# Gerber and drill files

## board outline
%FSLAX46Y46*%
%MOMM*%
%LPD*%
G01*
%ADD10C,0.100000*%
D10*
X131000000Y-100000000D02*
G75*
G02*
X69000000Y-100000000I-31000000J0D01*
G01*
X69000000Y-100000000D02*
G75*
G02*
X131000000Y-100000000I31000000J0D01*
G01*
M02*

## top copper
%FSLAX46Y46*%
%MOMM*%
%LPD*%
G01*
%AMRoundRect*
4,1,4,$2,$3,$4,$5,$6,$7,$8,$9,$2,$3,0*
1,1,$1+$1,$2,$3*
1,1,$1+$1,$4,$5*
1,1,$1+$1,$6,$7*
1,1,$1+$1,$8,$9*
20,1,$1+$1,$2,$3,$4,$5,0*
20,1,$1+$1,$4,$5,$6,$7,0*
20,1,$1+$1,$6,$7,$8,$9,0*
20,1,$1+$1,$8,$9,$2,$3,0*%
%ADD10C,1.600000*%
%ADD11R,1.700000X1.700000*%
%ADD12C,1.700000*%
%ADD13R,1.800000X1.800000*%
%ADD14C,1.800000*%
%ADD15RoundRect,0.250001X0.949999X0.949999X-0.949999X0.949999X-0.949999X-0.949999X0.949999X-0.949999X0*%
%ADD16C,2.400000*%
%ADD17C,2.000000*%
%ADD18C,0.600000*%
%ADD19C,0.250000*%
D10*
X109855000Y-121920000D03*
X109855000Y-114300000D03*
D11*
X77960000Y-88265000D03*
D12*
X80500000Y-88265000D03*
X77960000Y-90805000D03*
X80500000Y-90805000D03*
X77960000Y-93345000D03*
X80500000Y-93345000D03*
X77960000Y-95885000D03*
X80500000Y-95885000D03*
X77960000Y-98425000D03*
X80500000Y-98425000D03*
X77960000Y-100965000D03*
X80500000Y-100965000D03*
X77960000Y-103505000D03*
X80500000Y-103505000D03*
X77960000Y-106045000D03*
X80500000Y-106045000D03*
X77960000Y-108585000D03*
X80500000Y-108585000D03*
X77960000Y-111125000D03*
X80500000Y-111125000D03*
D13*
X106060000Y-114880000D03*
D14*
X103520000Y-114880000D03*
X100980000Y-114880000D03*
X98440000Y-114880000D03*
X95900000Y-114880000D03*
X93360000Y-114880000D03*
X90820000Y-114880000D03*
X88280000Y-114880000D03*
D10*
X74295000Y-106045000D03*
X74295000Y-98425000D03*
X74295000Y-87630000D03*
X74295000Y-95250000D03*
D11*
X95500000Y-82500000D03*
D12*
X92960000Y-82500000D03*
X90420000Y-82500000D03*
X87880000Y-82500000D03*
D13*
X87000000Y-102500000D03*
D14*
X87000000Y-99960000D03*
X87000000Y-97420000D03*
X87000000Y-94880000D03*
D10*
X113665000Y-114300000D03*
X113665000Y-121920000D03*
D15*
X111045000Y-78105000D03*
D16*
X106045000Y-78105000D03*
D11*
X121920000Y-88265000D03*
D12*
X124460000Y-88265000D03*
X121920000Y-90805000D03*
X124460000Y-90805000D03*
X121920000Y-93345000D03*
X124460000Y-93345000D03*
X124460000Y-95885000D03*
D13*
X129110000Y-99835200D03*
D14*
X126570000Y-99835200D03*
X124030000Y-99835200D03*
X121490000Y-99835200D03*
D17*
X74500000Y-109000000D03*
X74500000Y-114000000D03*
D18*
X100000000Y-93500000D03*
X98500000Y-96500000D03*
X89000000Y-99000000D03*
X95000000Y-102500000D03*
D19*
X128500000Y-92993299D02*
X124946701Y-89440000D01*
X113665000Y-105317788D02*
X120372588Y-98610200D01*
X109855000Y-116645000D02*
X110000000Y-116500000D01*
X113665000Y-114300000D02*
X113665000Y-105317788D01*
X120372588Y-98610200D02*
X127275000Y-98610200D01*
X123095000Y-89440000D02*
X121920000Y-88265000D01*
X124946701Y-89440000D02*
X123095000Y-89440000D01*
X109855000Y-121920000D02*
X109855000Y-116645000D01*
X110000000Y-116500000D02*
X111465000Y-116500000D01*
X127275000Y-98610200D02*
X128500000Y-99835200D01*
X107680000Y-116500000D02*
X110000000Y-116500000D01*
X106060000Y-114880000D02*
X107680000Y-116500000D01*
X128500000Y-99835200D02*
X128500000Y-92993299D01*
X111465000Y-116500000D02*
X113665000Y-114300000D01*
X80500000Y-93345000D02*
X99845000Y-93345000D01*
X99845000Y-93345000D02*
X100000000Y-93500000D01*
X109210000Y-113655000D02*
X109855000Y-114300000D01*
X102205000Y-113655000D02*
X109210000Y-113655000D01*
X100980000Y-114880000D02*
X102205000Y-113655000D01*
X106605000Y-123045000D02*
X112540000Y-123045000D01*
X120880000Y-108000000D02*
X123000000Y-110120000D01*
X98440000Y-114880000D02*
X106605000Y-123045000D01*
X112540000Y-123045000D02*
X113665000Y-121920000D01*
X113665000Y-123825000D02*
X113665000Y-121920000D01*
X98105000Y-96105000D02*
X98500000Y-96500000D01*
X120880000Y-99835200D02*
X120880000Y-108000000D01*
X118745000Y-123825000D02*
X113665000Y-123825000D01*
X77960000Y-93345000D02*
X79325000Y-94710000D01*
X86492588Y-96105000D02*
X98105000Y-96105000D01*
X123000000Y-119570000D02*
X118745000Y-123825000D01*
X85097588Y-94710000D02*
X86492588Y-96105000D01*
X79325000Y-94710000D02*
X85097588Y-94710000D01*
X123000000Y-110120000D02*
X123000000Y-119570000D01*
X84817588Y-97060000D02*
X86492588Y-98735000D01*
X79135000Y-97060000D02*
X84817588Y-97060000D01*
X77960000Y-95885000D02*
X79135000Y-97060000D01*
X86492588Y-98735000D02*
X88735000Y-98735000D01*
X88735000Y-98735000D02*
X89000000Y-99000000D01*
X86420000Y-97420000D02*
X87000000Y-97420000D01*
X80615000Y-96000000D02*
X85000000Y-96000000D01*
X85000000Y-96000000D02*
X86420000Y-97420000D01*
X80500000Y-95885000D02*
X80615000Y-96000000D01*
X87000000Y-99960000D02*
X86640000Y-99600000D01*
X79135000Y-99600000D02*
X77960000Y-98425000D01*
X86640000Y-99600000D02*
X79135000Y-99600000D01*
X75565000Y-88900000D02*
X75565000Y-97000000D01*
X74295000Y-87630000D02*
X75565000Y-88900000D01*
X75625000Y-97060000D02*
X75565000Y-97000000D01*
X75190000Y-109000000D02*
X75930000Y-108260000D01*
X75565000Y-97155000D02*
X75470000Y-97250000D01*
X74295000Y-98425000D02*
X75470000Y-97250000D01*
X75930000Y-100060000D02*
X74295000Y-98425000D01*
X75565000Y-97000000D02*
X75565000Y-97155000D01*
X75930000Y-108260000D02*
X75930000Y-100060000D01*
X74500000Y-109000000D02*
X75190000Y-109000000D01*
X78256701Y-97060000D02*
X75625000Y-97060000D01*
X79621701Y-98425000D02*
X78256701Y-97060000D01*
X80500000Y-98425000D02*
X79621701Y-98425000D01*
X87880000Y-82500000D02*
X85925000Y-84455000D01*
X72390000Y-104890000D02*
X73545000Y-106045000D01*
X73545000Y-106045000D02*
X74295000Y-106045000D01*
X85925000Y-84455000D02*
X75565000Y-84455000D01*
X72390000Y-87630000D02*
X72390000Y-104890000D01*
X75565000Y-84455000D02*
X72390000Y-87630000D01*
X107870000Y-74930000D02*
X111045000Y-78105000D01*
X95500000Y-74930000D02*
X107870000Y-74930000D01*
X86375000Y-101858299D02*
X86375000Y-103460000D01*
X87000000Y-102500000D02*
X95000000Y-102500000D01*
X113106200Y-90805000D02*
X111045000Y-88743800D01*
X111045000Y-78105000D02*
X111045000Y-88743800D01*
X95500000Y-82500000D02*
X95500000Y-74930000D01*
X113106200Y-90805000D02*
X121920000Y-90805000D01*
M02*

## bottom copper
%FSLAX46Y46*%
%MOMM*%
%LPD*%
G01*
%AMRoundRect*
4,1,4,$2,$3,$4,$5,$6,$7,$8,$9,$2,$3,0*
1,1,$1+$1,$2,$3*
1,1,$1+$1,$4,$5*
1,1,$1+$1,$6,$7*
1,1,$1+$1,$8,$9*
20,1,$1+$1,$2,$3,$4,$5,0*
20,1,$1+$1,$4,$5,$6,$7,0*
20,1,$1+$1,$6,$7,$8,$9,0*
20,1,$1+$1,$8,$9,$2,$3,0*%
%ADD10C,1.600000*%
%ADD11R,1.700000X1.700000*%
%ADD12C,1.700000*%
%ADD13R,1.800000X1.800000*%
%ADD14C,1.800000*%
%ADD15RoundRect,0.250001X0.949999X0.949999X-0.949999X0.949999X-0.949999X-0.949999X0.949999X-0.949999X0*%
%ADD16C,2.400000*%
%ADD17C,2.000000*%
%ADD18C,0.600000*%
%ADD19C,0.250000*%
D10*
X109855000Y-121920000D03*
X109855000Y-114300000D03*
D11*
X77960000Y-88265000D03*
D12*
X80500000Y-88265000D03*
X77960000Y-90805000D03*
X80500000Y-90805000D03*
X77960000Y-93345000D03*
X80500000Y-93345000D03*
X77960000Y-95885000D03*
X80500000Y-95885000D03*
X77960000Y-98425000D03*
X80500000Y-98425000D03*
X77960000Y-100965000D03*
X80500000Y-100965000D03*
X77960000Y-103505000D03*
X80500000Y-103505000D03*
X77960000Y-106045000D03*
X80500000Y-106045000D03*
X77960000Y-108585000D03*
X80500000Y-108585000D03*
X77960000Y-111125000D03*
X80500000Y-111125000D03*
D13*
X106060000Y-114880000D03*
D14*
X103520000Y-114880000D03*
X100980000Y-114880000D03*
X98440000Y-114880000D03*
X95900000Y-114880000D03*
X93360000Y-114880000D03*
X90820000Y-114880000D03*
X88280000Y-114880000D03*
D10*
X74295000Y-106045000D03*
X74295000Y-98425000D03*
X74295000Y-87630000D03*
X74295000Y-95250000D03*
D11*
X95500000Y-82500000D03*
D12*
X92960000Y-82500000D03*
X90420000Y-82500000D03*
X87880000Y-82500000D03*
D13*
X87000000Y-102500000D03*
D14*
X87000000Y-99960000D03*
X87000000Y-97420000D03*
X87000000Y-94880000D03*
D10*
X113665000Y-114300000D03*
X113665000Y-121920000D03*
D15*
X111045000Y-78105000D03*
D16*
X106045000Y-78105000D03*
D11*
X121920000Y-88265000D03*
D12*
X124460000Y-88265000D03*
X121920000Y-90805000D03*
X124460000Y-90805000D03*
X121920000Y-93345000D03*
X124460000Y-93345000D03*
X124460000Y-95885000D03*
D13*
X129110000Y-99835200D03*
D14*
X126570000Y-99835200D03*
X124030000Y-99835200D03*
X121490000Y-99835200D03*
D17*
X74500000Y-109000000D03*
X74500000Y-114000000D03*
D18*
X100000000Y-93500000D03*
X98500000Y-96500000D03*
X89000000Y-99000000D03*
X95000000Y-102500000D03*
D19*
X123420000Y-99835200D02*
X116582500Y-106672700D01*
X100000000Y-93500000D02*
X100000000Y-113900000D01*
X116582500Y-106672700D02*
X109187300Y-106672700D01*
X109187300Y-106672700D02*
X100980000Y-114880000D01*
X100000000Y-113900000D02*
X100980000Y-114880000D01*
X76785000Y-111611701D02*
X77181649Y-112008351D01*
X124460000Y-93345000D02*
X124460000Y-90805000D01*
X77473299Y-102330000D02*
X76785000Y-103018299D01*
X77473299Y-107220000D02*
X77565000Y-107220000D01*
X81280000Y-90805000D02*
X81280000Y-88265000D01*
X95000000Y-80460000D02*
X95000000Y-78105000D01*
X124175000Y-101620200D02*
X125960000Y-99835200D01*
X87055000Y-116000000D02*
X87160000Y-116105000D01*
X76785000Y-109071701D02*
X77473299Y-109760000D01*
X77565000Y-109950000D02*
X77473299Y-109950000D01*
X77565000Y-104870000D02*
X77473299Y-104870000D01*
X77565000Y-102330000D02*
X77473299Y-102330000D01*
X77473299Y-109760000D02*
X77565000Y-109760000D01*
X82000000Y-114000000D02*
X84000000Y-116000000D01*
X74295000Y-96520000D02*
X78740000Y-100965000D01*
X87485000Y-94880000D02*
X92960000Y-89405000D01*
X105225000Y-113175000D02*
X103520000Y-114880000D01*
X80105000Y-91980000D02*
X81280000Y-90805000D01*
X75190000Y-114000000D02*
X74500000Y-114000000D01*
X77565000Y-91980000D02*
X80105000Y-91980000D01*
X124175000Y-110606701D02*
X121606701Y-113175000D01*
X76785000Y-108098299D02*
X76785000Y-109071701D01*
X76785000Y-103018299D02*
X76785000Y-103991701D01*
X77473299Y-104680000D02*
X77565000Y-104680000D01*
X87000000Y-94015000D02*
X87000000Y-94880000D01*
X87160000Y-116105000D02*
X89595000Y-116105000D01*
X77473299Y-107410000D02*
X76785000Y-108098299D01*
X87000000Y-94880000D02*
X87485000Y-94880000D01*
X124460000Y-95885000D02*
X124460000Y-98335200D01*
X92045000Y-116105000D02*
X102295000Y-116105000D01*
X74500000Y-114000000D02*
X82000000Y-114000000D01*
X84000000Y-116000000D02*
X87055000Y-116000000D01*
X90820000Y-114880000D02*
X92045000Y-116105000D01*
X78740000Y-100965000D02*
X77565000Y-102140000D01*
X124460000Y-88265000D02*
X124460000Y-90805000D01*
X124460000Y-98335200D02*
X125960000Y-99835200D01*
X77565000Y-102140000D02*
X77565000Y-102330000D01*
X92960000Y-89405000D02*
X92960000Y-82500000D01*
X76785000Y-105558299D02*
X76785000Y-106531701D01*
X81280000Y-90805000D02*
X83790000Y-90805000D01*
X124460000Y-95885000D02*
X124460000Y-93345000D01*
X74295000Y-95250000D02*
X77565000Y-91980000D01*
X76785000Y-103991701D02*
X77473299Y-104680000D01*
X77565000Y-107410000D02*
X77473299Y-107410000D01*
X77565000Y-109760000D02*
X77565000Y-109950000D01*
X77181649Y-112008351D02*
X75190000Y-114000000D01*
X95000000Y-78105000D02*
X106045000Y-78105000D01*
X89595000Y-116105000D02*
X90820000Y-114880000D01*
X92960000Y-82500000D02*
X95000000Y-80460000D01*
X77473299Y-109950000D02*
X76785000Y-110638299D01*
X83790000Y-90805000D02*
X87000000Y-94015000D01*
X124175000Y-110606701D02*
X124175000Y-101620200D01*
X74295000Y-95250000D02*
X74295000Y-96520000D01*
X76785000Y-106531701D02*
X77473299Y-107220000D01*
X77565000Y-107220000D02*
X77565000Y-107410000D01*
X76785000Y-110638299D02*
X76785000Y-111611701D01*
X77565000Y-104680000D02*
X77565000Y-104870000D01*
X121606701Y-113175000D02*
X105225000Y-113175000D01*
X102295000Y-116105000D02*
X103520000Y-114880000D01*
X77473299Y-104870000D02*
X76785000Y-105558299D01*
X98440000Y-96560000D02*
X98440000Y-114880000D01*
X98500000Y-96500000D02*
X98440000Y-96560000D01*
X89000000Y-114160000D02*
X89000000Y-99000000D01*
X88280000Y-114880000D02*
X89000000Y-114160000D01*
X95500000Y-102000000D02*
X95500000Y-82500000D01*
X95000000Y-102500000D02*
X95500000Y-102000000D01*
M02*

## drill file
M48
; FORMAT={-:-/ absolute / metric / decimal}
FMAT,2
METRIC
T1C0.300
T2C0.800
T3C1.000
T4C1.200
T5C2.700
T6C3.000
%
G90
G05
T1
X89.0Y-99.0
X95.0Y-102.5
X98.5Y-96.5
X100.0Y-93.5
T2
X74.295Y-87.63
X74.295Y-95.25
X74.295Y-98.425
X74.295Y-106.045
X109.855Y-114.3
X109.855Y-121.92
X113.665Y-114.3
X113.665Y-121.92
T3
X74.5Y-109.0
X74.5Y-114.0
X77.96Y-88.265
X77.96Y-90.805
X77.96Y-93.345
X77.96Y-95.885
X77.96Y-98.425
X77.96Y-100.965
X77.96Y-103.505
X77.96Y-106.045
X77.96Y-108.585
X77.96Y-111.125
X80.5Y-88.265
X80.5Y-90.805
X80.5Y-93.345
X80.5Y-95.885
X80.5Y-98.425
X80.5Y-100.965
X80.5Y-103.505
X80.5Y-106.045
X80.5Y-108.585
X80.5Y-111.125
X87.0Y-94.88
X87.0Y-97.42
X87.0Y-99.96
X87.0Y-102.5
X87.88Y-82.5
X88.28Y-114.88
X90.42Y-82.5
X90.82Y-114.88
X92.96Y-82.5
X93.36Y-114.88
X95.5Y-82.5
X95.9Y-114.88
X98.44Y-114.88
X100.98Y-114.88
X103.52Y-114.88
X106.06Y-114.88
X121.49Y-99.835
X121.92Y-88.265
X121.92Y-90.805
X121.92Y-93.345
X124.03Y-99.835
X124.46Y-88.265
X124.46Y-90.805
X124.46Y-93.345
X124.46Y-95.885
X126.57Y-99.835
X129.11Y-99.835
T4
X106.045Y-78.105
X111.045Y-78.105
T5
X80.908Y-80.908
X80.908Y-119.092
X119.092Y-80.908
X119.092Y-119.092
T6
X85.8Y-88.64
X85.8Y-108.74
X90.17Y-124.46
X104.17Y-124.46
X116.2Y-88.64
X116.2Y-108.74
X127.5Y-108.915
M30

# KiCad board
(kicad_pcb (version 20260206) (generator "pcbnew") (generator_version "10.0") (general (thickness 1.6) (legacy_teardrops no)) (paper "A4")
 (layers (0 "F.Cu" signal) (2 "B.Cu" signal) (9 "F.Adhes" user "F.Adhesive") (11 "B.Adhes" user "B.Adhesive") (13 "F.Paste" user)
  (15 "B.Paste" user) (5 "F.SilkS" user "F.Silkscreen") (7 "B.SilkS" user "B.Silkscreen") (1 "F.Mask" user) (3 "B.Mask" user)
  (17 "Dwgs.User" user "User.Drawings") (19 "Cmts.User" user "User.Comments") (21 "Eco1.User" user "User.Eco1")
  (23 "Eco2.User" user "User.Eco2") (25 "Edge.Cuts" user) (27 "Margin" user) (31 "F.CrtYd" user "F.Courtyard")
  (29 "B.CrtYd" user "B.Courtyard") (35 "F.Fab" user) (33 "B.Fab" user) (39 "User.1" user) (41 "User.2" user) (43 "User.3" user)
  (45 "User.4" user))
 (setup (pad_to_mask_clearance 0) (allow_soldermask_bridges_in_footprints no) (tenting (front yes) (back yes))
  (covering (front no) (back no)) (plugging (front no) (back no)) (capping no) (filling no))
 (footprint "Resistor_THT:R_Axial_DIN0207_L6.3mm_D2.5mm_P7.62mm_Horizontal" (layer "F.Cu") (at 109.855 121.92 90)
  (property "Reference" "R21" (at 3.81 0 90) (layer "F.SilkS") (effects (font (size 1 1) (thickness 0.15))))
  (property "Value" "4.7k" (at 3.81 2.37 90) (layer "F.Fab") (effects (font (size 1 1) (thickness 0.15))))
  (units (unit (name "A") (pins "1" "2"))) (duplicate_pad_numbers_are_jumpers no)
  (pad "1" thru_hole circle (at 0 0 90) (size 1.6 1.6) (drill 0.8) (layers "*.Cu" "*.Mask") (remove_unused_layers no) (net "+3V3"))
  (pad "2" thru_hole circle (at 7.62 0 90) (size 1.6 1.6) (drill 0.8) (layers "*.Cu" "*.Mask") (remove_unused_layers no) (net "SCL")))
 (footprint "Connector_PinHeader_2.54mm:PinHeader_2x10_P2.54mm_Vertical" (layer "F.Cu") (at 77.96 88.265)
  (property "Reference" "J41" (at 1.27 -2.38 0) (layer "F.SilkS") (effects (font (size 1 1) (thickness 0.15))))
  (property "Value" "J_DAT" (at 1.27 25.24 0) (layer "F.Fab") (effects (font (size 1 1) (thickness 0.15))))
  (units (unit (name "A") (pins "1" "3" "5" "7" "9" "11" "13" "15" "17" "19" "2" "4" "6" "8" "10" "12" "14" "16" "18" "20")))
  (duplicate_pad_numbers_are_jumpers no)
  (pad "1" thru_hole rect (at 0 0) (size 1.7 1.7) (drill 1) (layers "*.Cu" "*.Mask") (remove_unused_layers no)
   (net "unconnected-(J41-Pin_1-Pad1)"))
  (pad "2" thru_hole circle (at 2.54 0) (size 1.7 1.7) (drill 1) (layers "*.Cu" "*.Mask") (remove_unused_layers no) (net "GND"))
  (pad "3" thru_hole circle (at 0 2.54) (size 1.7 1.7) (drill 1) (layers "*.Cu" "*.Mask") (remove_unused_layers no)
   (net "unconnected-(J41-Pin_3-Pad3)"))
  (pad "4" thru_hole circle (at 2.54 2.54) (size 1.7 1.7) (drill 1) (layers "*.Cu" "*.Mask") (remove_unused_layers no) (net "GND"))
  (pad "5" thru_hole circle (at 0 5.08) (size 1.7 1.7) (drill 1) (layers "*.Cu" "*.Mask") (remove_unused_layers no) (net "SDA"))
  (pad "6" thru_hole circle (at 2.54 5.08) (size 1.7 1.7) (drill 1) (layers "*.Cu" "*.Mask") (remove_unused_layers no) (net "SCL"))
  (pad "7" thru_hole circle (at 0 7.62) (size 1.7 1.7) (drill 1) (layers "*.Cu" "*.Mask") (remove_unused_layers no) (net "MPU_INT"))
  (pad "8" thru_hole circle (at 2.54 7.62) (size 1.7 1.7) (drill 1) (layers "*.Cu" "*.Mask") (remove_unused_layers no) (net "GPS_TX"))
  (pad "9" thru_hole circle (at 0 10.16) (size 1.7 1.7) (drill 1) (layers "*.Cu" "*.Mask") (remove_unused_layers no) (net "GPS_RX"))
  (pad "10" thru_hole circle (at 2.54 10.16) (size 1.7 1.7) (drill 1) (layers "*.Cu" "*.Mask") (remove_unused_layers no) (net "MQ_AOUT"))
  (pad "11" thru_hole circle (at 0 12.7) (size 1.7 1.7) (drill 1) (layers "*.Cu" "*.Mask") (remove_unused_layers no) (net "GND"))
  (pad "12" thru_hole circle (at 2.54 12.7) (size 1.7 1.7) (drill 1) (layers "*.Cu" "*.Mask") (remove_unused_layers no)
   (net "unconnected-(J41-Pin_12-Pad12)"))
  (pad "13" thru_hole circle (at 0 15.24) (size 1.7 1.7) (drill 1) (layers "*.Cu" "*.Mask") (remove_unused_layers no)
   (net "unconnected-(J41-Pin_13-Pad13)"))
  (pad "14" thru_hole circle (at 2.54 15.24) (size 1.7 1.7) (drill 1) (layers "*.Cu" "*.Mask") (remove_unused_layers no)
   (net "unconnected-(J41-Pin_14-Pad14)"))
  (pad "15" thru_hole circle (at 0 17.78) (size 1.7 1.7) (drill 1) (layers "*.Cu" "*.Mask") (remove_unused_layers no)
   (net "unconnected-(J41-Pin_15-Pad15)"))
  (pad "16" thru_hole circle (at 2.54 17.78) (size 1.7 1.7) (drill 1) (layers "*.Cu" "*.Mask") (remove_unused_layers no)
   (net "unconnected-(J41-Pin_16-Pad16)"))
  (pad "17" thru_hole circle (at 0 20.32) (size 1.7 1.7) (drill 1) (layers "*.Cu" "*.Mask") (remove_unused_layers no)
   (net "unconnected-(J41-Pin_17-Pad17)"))
  (pad "18" thru_hole circle (at 2.54 20.32) (size 1.7 1.7) (drill 1) (layers "*.Cu" "*.Mask") (remove_unused_layers no)
   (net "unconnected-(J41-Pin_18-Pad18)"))
  (pad "19" thru_hole circle (at 0 22.86) (size 1.7 1.7) (drill 1) (layers "*.Cu" "*.Mask") (remove_unused_layers no)
   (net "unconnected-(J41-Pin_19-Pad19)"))
  (pad "20" thru_hole circle (at 2.54 22.86) (size 1.7 1.7) (drill 1) (layers "*.Cu" "*.Mask") (remove_unused_layers no)
   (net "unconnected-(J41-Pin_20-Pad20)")))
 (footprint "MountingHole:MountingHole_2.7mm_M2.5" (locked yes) (layer "F.Cu") (at 119.092 119.092)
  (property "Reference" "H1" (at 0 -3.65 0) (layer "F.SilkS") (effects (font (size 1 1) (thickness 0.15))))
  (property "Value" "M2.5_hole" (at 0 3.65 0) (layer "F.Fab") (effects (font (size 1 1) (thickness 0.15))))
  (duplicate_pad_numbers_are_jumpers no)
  (pad "" np_thru_hole circle (at 0 0) (size 2.7 2.7) (drill 2.7) (layers "*.Cu" "*.Mask")))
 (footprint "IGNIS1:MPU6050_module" (layer "F.Cu") (at 97.17 119.96 -90)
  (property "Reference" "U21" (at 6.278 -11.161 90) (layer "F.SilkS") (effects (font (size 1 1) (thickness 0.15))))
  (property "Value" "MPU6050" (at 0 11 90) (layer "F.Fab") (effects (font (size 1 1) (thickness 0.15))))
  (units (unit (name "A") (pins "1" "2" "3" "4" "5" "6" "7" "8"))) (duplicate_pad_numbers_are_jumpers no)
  (pad "" np_thru_hole circle (at 4.5 -7 270) (size 3 3) (drill 3) (layers "*.Cu" "*.Mask"))
  (pad "" np_thru_hole circle (at 4.5 7 270) (size 3 3) (drill 3) (layers "*.Cu" "*.Mask"))
  (pad "1" thru_hole rect (at -5.08 -8.89 270) (size 1.8 1.8) (drill 1) (layers "*.Cu" "*.Mask") (remove_unused_layers no) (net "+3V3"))
  (pad "2" thru_hole circle (at -5.08 -6.35 270) (size 1.8 1.8) (drill 1) (layers "*.Cu" "*.Mask") (remove_unused_layers no) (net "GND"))
  (pad "3" thru_hole circle (at -5.08 -3.81 270) (size 1.8 1.8) (drill 1) (layers "*.Cu" "*.Mask") (remove_unused_layers no) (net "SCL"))
  (pad "4" thru_hole circle (at -5.08 -1.27 270) (size 1.8 1.8) (drill 1) (layers "*.Cu" "*.Mask") (remove_unused_layers no) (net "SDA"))
  (pad "5" thru_hole circle (at -5.08 1.27 270) (size 1.8 1.8) (drill 1) (layers "*.Cu" "*.Mask") (remove_unused_layers no)
   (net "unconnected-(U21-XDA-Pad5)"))
  (pad "6" thru_hole circle (at -5.08 3.81 270) (size 1.8 1.8) (drill 1) (layers "*.Cu" "*.Mask") (remove_unused_layers no)
   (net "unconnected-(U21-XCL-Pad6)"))
  (pad "7" thru_hole circle (at -5.08 6.35 270) (size 1.8 1.8) (drill 1) (layers "*.Cu" "*.Mask") (remove_unused_layers no) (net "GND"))
  (pad "8" thru_hole circle (at -5.08 8.89 270) (size 1.8 1.8) (drill 1) (layers "*.Cu" "*.Mask") (remove_unused_layers no) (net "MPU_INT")))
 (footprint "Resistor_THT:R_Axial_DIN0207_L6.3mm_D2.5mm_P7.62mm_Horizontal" (layer "F.Cu") (at 74.295 106.045 90)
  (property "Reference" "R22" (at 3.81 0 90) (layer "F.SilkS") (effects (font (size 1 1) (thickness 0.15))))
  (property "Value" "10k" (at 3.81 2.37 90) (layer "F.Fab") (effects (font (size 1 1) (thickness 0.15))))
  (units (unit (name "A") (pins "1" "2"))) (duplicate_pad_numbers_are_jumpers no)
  (pad "1" thru_hole circle (at 0 0 90) (size 1.6 1.6) (drill 0.8) (layers "*.Cu" "*.Mask") (remove_unused_layers no) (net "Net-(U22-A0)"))
  (pad "2" thru_hole circle (at 7.62 0 90) (size 1.6 1.6) (drill 0.8) (layers "*.Cu" "*.Mask") (remove_unused_layers no) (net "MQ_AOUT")))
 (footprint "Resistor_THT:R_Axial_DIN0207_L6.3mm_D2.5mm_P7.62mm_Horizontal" (layer "F.Cu") (at 74.295 87.63 -90)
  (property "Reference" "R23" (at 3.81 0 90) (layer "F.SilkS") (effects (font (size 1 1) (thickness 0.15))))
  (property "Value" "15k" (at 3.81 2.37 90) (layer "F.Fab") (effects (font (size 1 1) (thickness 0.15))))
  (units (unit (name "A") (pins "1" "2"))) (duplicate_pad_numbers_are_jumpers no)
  (pad "1" thru_hole circle (at 0 0 270) (size 1.6 1.6) (drill 0.8) (layers "*.Cu" "*.Mask") (remove_unused_layers no) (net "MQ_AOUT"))
  (pad "2" thru_hole circle (at 7.62 0 270) (size 1.6 1.6) (drill 0.8) (layers "*.Cu" "*.Mask") (remove_unused_layers no) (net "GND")))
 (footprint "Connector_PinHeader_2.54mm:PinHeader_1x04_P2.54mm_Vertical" (layer "F.Cu") (at 95.5 82.5 -90)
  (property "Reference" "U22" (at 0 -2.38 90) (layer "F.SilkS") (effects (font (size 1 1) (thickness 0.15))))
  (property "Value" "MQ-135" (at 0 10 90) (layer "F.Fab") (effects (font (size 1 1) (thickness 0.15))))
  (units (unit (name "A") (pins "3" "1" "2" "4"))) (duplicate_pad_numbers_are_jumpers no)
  (pad "1" thru_hole rect (at 0 0 270) (size 1.7 1.7) (drill 1) (layers "*.Cu" "*.Mask") (remove_unused_layers no) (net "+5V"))
  (pad "2" thru_hole circle (at 0 2.54 270) (size 1.7 1.7) (drill 1) (layers "*.Cu" "*.Mask") (remove_unused_layers no) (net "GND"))
  (pad "3" thru_hole circle (at 0 5.08 270) (size 1.7 1.7) (drill 1) (layers "*.Cu" "*.Mask") (remove_unused_layers no)
   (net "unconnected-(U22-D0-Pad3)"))
  (pad "4" thru_hole circle (at 0 7.62 270) (size 1.7 1.7) (drill 1) (layers "*.Cu" "*.Mask") (remove_unused_layers no) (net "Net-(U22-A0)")))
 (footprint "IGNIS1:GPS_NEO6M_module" (layer "F.Cu") (at 101 98.69)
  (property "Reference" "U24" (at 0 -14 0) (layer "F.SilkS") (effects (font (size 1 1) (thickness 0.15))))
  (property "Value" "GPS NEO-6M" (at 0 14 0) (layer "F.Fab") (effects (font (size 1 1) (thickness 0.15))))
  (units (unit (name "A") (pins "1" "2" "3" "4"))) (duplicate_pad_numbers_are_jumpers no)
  (pad "" np_thru_hole circle (at -15.2 -10.05) (size 3 3) (drill 3) (layers "*.Cu" "*.Mask"))
  (pad "" np_thru_hole circle (at -15.2 10.05) (size 3 3) (drill 3) (layers "*.Cu" "*.Mask"))
  (pad "" np_thru_hole circle (at 15.2 -10.05) (size 3 3) (drill 3) (layers "*.Cu" "*.Mask"))
  (pad "" np_thru_hole circle (at 15.2 10.05) (size 3 3) (drill 3) (layers "*.Cu" "*.Mask"))
  (pad "1" thru_hole rect (at -14 3.81) (size 1.8 1.8) (drill 1) (layers "*.Cu" "*.Mask") (remove_unused_layers no) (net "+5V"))
  (pad "2" thru_hole circle (at -14 1.27) (size 1.8 1.8) (drill 1) (layers "*.Cu" "*.Mask") (remove_unused_layers no) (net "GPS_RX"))
  (pad "3" thru_hole circle (at -14 -1.27) (size 1.8 1.8) (drill 1) (layers "*.Cu" "*.Mask") (remove_unused_layers no) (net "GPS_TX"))
  (pad "4" thru_hole circle (at -14 -3.81) (size 1.8 1.8) (drill 1) (layers "*.Cu" "*.Mask") (remove_unused_layers no) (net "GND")))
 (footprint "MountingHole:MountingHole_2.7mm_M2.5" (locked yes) (layer "F.Cu") (at 80.908 80.908)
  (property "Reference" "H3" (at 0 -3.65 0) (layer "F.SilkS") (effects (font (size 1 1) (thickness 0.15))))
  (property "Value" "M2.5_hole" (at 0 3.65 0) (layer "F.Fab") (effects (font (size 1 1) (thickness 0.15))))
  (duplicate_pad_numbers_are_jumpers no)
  (pad "" np_thru_hole circle (at 0 0) (size 2.7 2.7) (drill 2.7) (layers "*.Cu" "*.Mask")))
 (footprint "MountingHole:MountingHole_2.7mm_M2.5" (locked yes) (layer "F.Cu") (at 119.092 80.908)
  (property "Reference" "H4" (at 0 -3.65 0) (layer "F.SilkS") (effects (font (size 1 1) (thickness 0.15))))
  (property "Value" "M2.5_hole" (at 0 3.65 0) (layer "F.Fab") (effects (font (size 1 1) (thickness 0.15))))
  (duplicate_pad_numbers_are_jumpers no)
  (pad "" np_thru_hole circle (at 0 0) (size 2.7 2.7) (drill 2.7) (layers "*.Cu" "*.Mask")))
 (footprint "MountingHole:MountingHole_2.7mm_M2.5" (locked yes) (layer "F.Cu") (at 80.908 119.092)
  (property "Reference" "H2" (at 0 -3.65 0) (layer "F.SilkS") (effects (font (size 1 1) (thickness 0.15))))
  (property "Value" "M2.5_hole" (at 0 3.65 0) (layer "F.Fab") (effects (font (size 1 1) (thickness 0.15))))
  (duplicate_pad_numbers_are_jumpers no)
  (pad "" np_thru_hole circle (at 0 0) (size 2.7 2.7) (drill 2.7) (layers "*.Cu" "*.Mask")))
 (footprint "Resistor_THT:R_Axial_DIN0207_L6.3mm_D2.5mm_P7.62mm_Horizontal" (layer "F.Cu") (at 113.665 114.3 -90)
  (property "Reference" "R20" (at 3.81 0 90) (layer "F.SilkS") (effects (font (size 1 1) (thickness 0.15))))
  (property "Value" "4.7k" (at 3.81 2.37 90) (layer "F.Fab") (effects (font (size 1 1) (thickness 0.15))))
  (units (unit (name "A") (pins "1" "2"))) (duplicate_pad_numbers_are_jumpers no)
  (pad "1" thru_hole circle (at 0 0 270) (size 1.6 1.6) (drill 0.8) (layers "*.Cu" "*.Mask") (remove_unused_layers no) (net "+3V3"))
  (pad "2" thru_hole circle (at 7.62 0 270) (size 1.6 1.6) (drill 0.8) (layers "*.Cu" "*.Mask") (remove_unused_layers no) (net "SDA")))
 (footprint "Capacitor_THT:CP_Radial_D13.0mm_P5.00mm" (layer "F.Cu") (at 111.045 78.105 180)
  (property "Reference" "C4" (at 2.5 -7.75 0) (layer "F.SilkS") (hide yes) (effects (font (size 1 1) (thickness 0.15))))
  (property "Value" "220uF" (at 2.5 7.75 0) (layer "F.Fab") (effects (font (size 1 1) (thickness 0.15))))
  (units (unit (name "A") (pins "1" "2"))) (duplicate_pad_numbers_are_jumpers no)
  (pad "1" thru_hole roundrect (at 0 0 180) (size 2.4 2.4) (drill 1.2) (layers "*.Cu" "*.Mask") (remove_unused_layers no)
   (roundrect_rratio 0.104167) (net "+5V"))
  (pad "2" thru_hole circle (at 5 0 180) (size 2.4 2.4) (drill 1.2) (layers "*.Cu" "*.Mask") (remove_unused_layers no) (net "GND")))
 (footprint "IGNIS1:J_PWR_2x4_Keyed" (layer "F.Cu") (at 123.19 92.075)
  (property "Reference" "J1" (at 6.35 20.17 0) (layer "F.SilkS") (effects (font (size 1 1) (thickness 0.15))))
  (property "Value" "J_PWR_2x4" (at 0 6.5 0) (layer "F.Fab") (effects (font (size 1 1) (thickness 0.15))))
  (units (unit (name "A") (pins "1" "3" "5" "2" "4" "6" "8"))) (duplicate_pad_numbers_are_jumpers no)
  (pad "1" thru_hole rect (at -1.27 -3.81) (size 1.7 1.7) (drill 1) (layers "*.Cu" "*.Mask") (remove_unused_layers no) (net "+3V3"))
  (pad "2" thru_hole circle (at 1.27 -3.81) (size 1.7 1.7) (drill 1) (layers "*.Cu" "*.Mask") (remove_unused_layers no) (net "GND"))
  (pad "3" thru_hole circle (at -1.27 -1.27) (size 1.7 1.7) (drill 1) (layers "*.Cu" "*.Mask") (remove_unused_layers no) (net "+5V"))
  (pad "4" thru_hole circle (at 1.27 -1.27) (size 1.7 1.7) (drill 1) (layers "*.Cu" "*.Mask") (remove_unused_layers no) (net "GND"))
  (pad "5" thru_hole circle (at -1.27 1.27) (size 1.7 1.7) (drill 1) (layers "*.Cu" "*.Mask") (remove_unused_layers no)
   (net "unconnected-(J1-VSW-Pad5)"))
  (pad "6" thru_hole circle (at 1.27 1.27) (size 1.7 1.7) (drill 1) (layers "*.Cu" "*.Mask") (remove_unused_layers no) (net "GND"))
  (pad "8" thru_hole circle (at 1.27 3.81) (size 1.7 1.7) (drill 1) (layers "*.Cu" "*.Mask") (remove_unused_layers no) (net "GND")))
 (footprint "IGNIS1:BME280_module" (layer "F.Cu") (at 125.3 104.9152 -90)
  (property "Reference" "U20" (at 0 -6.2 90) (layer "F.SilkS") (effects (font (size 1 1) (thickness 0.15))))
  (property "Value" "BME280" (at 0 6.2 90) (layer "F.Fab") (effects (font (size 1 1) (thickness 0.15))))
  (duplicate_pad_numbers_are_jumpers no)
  (pad "" np_thru_hole circle (at 4 -2.2 270) (size 3 3) (drill 3) (layers "*.Cu" "*.Mask"))
  (pad "1" thru_hole rect (at -5.08 -3.81 270) (size 1.8 1.8) (drill 1) (layers "*.Cu" "*.Mask") (remove_unused_layers no) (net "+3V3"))
  (pad "2" thru_hole circle (at -5.08 -1.27 270) (size 1.8 1.8) (drill 1) (layers "*.Cu" "*.Mask") (remove_unused_layers no) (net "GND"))
  (pad "3" thru_hole circle (at -5.08 1.27 270) (size 1.8 1.8) (drill 1) (layers "*.Cu" "*.Mask") (remove_unused_layers no) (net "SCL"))
  (pad "4" thru_hole circle (at -5.08 3.81 270) (size 1.8 1.8) (drill 1) (layers "*.Cu" "*.Mask") (remove_unused_layers no) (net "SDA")))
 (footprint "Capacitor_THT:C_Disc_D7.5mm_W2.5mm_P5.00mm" (layer "F.Cu") (at 74.5 109 -90)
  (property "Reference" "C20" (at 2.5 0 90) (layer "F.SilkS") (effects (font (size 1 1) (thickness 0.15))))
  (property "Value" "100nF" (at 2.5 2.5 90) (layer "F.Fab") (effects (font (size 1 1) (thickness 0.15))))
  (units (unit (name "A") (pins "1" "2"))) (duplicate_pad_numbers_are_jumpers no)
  (pad "1" thru_hole circle (at 0 0 270) (size 2 2) (drill 1) (layers "*.Cu" "*.Mask") (remove_unused_layers no) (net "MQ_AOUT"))
  (pad "2" thru_hole circle (at 5 0 270) (size 2 2) (drill 1) (layers "*.Cu" "*.Mask") (remove_unused_layers no) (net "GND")))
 (gr_circle (center 100 100) (end 131 100) (stroke (width 0.1) (type solid)) (fill no) (locked yes) (layer "Edge.Cuts"))
 (segment (start 128.5 92.993299) (end 124.946701 89.44) (width 0.25) (layer "F.Cu") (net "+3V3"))
 (segment (start 113.665 105.317788) (end 120.372588 98.6102) (width 0.25) (layer "F.Cu") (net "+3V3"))
 (segment (start 109.855 116.645) (end 110 116.5) (width 0.25) (layer "F.Cu") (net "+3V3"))
 (segment (start 113.665 114.3) (end 113.665 105.317788) (width 0.25) (layer "F.Cu") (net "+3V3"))
 (segment (start 120.372588 98.6102) (end 127.275 98.6102) (width 0.25) (layer "F.Cu") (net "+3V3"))
 (segment (start 123.095 89.44) (end 121.92 88.265) (width 0.25) (layer "F.Cu") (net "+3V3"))
 (segment (start 124.946701 89.44) (end 123.095 89.44) (width 0.25) (layer "F.Cu") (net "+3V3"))
 (segment (start 109.855 121.92) (end 109.855 116.645) (width 0.25) (layer "F.Cu") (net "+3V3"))
 (segment (start 110 116.5) (end 111.465 116.5) (width 0.25) (layer "F.Cu") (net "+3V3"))
 (segment (start 127.275 98.6102) (end 128.5 99.8352) (width 0.25) (layer "F.Cu") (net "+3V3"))
 (segment (start 107.68 116.5) (end 110 116.5) (width 0.25) (layer "F.Cu") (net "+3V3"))
 (segment (start 106.06 114.88) (end 107.68 116.5) (width 0.25) (layer "F.Cu") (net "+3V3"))
 (segment (start 128.5 99.8352) (end 128.5 92.993299) (width 0.25) (layer "F.Cu") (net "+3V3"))
 (segment (start 111.465 116.5) (end 113.665 114.3) (width 0.25) (layer "F.Cu") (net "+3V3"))
 (segment (start 80.5 93.345) (end 99.845 93.345) (width 0.25) (layer "F.Cu") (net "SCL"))
 (segment (start 99.845 93.345) (end 100 93.5) (width 0.25) (layer "F.Cu") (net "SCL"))
 (segment (start 109.21 113.655) (end 109.855 114.3) (width 0.25) (layer "F.Cu") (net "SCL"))
 (segment (start 102.205 113.655) (end 109.21 113.655) (width 0.25) (layer "F.Cu") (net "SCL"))
 (segment (start 100.98 114.88) (end 102.205 113.655) (width 0.25) (layer "F.Cu") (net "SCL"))
 (via (at 100 93.5) (size 0.6) (drill 0.3) (layers "F.Cu" "B.Cu") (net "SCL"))
 (segment (start 123.42 99.8352) (end 116.5825 106.6727) (width 0.25) (layer "B.Cu") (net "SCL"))
 (segment (start 100 93.5) (end 100 113.9) (width 0.25) (layer "B.Cu") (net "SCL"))
 (segment (start 116.5825 106.6727) (end 109.1873 106.6727) (width 0.25) (layer "B.Cu") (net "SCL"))
 (segment (start 109.1873 106.6727) (end 100.98 114.88) (width 0.25) (layer "B.Cu") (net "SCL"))
 (segment (start 100 113.9) (end 100.98 114.88) (width 0.25) (layer "B.Cu") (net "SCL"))
 (segment (start 76.785 111.611701) (end 77.181649 112.008351) (width 0.25) (layer "B.Cu") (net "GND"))
 (segment (start 124.46 93.345) (end 124.46 90.805) (width 0.25) (layer "B.Cu") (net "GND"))
 (segment (start 77.473299 102.33) (end 76.785 103.018299) (width 0.25) (layer "B.Cu") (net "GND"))
 (segment (start 77.473299 107.22) (end 77.565 107.22) (width 0.25) (layer "B.Cu") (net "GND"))
 (segment (start 81.28 90.805) (end 81.28 88.265) (width 0.25) (layer "B.Cu") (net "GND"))
 (segment (start 95 80.46) (end 95 78.105) (width 0.25) (layer "B.Cu") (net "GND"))
 (segment (start 124.175 101.6202) (end 125.96 99.8352) (width 0.25) (layer "B.Cu") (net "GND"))
 (segment (start 87.055 116) (end 87.16 116.105) (width 0.25) (layer "B.Cu") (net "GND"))
 (segment (start 76.785 109.071701) (end 77.473299 109.76) (width 0.25) (layer "B.Cu") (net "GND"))
 (segment (start 77.565 109.95) (end 77.473299 109.95) (width 0.25) (layer "B.Cu") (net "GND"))
 (segment (start 77.565 104.87) (end 77.473299 104.87) (width 0.25) (layer "B.Cu") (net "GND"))
 (segment (start 77.565 102.33) (end 77.473299 102.33) (width 0.25) (layer "B.Cu") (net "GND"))
 (segment (start 77.473299 109.76) (end 77.565 109.76) (width 0.25) (layer "B.Cu") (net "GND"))
 (segment (start 82 114) (end 84 116) (width 0.25) (layer "B.Cu") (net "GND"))
 (segment (start 74.295 96.52) (end 78.74 100.965) (width 0.25) (layer "B.Cu") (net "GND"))
 (segment (start 87.485 94.88) (end 92.96 89.405) (width 0.25) (layer "B.Cu") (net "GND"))
 (segment (start 105.225 113.175) (end 103.52 114.88) (width 0.25) (layer "B.Cu") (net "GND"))
 (segment (start 80.105 91.98) (end 81.28 90.805) (width 0.25) (layer "B.Cu") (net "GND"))
 (segment (start 75.19 114) (end 74.5 114) (width 0.25) (layer "B.Cu") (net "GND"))
 (segment (start 77.565 91.98) (end 80.105 91.98) (width 0.25) (layer "B.Cu") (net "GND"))
 (segment (start 124.175 110.606701) (end 121.606701 113.175) (width 0.25) (layer "B.Cu") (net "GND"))
 (segment (start 76.785 108.098299) (end 76.785 109.071701) (width 0.25) (layer "B.Cu") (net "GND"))
 (segment (start 76.785 103.018299) (end 76.785 103.991701) (width 0.25) (layer "B.Cu") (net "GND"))
 (segment (start 77.473299 104.68) (end 77.565 104.68) (width 0.25) (layer "B.Cu") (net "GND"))
 (segment (start 87 94.015) (end 87 94.88) (width 0.25) (layer "B.Cu") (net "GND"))
 (segment (start 87.16 116.105) (end 89.595 116.105) (width 0.25) (layer "B.Cu") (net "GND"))
 (segment (start 77.473299 107.41) (end 76.785 108.098299) (width 0.25) (layer "B.Cu") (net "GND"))
 (segment (start 87 94.88) (end 87.485 94.88) (width 0.25) (layer "B.Cu") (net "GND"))
 (segment (start 124.46 95.885) (end 124.46 98.3352) (width 0.25) (layer "B.Cu") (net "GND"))
 (segment (start 92.045 116.105) (end 102.295 116.105) (width 0.25) (layer "B.Cu") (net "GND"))
 (segment (start 74.5 114) (end 82 114) (width 0.25) (layer "B.Cu") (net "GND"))
 (segment (start 84 116) (end 87.055 116) (width 0.25) (layer "B.Cu") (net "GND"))
 (segment (start 90.82 114.88) (end 92.045 116.105) (width 0.25) (layer "B.Cu") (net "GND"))
 (segment (start 78.74 100.965) (end 77.565 102.14) (width 0.25) (layer "B.Cu") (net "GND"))
 (segment (start 124.46 88.265) (end 124.46 90.805) (width 0.25) (layer "B.Cu") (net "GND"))
 (segment (start 124.46 98.3352) (end 125.96 99.8352) (width 0.25) (layer "B.Cu") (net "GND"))
 (segment (start 77.565 102.14) (end 77.565 102.33) (width 0.25) (layer "B.Cu") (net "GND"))
 (segment (start 92.96 89.405) (end 92.96 82.5) (width 0.25) (layer "B.Cu") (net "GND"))
 (segment (start 76.785 105.558299) (end 76.785 106.531701) (width 0.25) (layer "B.Cu") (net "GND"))
 (segment (start 81.28 90.805) (end 83.79 90.805) (width 0.25) (layer "B.Cu") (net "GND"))
 (segment (start 124.46 95.885) (end 124.46 93.345) (width 0.25) (layer "B.Cu") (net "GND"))
 (segment (start 74.295 95.25) (end 77.565 91.98) (width 0.25) (layer "B.Cu") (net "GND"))
 (segment (start 76.785 103.991701) (end 77.473299 104.68) (width 0.25) (layer "B.Cu") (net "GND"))
 (segment (start 77.565 107.41) (end 77.473299 107.41) (width 0.25) (layer "B.Cu") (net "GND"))
 (segment (start 77.565 109.76) (end 77.565 109.95) (width 0.25) (layer "B.Cu") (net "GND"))
 (segment (start 77.181649 112.008351) (end 75.19 114) (width 0.25) (layer "B.Cu") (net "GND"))
 (segment (start 95 78.105) (end 106.045 78.105) (width 0.25) (layer "B.Cu") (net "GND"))
 (segment (start 89.595 116.105) (end 90.82 114.88) (width 0.25) (layer "B.Cu") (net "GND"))
 (segment (start 92.96 82.5) (end 95 80.46) (width 0.25) (layer "B.Cu") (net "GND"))
 (segment (start 77.473299 109.95) (end 76.785 110.638299) (width 0.25) (layer "B.Cu") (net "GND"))
 (segment (start 83.79 90.805) (end 87 94.015) (width 0.25) (layer "B.Cu") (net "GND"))
 (segment (start 124.175 110.606701) (end 124.175 101.6202) (width 0.25) (layer "B.Cu") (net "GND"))
 (segment (start 74.295 95.25) (end 74.295 96.52) (width 0.25) (layer "B.Cu") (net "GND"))
 (segment (start 76.785 106.531701) (end 77.473299 107.22) (width 0.25) (layer "B.Cu") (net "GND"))
 (segment (start 77.565 107.22) (end 77.565 107.41) (width 0.25) (layer "B.Cu") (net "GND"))
 (segment (start 76.785 110.638299) (end 76.785 111.611701) (width 0.25) (layer "B.Cu") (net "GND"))
 (segment (start 77.565 104.68) (end 77.565 104.87) (width 0.25) (layer "B.Cu") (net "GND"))
 (segment (start 121.606701 113.175) (end 105.225 113.175) (width 0.25) (layer "B.Cu") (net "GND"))
 (segment (start 102.295 116.105) (end 103.52 114.88) (width 0.25) (layer "B.Cu") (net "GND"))
 (segment (start 77.473299 104.87) (end 76.785 105.558299) (width 0.25) (layer "B.Cu") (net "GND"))
 (segment (start 106.605 123.045) (end 112.54 123.045) (width 0.25) (layer "F.Cu") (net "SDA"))
 (segment (start 120.88 108) (end 123 110.12) (width 0.25) (layer "F.Cu") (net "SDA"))
 (segment (start 98.44 114.88) (end 106.605 123.045) (width 0.25) (layer "F.Cu") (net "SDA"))
 (segment (start 112.54 123.045) (end 113.665 121.92) (width 0.25) (layer "F.Cu") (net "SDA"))
 (segment (start 113.665 123.825) (end 113.665 121.92) (width 0.25) (layer "F.Cu") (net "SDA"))
 (segment (start 98.105 96.105) (end 98.5 96.5) (width 0.25) (layer "F.Cu") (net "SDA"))
 (segment (start 120.88 99.8352) (end 120.88 108) (width 0.25) (layer "F.Cu") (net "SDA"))
 (segment (start 118.745 123.825) (end 113.665 123.825) (width 0.25) (layer "F.Cu") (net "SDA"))
 (segment (start 77.96 93.345) (end 79.325 94.71) (width 0.25) (layer "F.Cu") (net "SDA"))
 (segment (start 86.492588 96.105) (end 98.105 96.105) (width 0.25) (layer "F.Cu") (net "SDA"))
 (segment (start 123 119.57) (end 118.745 123.825) (width 0.25) (layer "F.Cu") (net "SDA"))
 (segment (start 85.097588 94.71) (end 86.492588 96.105) (width 0.25) (layer "F.Cu") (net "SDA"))
 (segment (start 79.325 94.71) (end 85.097588 94.71) (width 0.25) (layer "F.Cu") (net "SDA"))
 (segment (start 123 110.12) (end 123 119.57) (width 0.25) (layer "F.Cu") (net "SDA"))
 (via (at 98.5 96.5) (size 0.6) (drill 0.3) (layers "F.Cu" "B.Cu") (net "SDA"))
 (segment (start 98.44 96.56) (end 98.44 114.88) (width 0.25) (layer "B.Cu") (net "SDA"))
 (segment (start 98.5 96.5) (end 98.44 96.56) (width 0.25) (layer "B.Cu") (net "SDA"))
 (segment (start 84.817588 97.06) (end 86.492588 98.735) (width 0.25) (layer "F.Cu") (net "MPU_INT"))
 (segment (start 79.135 97.06) (end 84.817588 97.06) (width 0.25) (layer "F.Cu") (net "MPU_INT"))
 (segment (start 77.96 95.885) (end 79.135 97.06) (width 0.25) (layer "F.Cu") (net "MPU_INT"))
 (segment (start 86.492588 98.735) (end 88.735 98.735) (width 0.25) (layer "F.Cu") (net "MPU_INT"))
 (segment (start 88.735 98.735) (end 89 99) (width 0.25) (layer "F.Cu") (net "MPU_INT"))
 (via (at 89 99) (size 0.6) (drill 0.3) (layers "F.Cu" "B.Cu") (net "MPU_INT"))
 (segment (start 89 114.16) (end 89 99) (width 0.25) (layer "B.Cu") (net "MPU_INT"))
 (segment (start 88.28 114.88) (end 89 114.16) (width 0.25) (layer "B.Cu") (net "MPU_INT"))
 (segment (start 86.42 97.42) (end 87 97.42) (width 0.25) (layer "F.Cu") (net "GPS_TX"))
 (segment (start 80.615 96) (end 85 96) (width 0.25) (layer "F.Cu") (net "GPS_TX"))
 (segment (start 85 96) (end 86.42 97.42) (width 0.25) (layer "F.Cu") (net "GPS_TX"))
 (segment (start 80.5 95.885) (end 80.615 96) (width 0.25) (layer "F.Cu") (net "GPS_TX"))
 (segment (start 87 99.96) (end 86.64 99.6) (width 0.25) (layer "F.Cu") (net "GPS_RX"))
 (segment (start 79.135 99.6) (end 77.96 98.425) (width 0.25) (layer "F.Cu") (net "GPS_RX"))
 (segment (start 86.64 99.6) (end 79.135 99.6) (width 0.25) (layer "F.Cu") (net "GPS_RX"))
 (segment (start 75.565 88.9) (end 75.565 97) (width 0.25) (layer "F.Cu") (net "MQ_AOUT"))
 (segment (start 74.295 87.63) (end 75.565 88.9) (width 0.25) (layer "F.Cu") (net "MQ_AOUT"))
 (segment (start 75.625 97.06) (end 75.565 97) (width 0.25) (layer "F.Cu") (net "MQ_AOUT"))
 (segment (start 75.19 109) (end 75.93 108.26) (width 0.25) (layer "F.Cu") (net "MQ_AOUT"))
 (segment (start 75.565 97.155) (end 75.47 97.25) (width 0.25) (layer "F.Cu") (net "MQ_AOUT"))
 (segment (start 74.295 98.425) (end 75.47 97.25) (width 0.25) (layer "F.Cu") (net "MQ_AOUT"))
 (segment (start 75.93 100.06) (end 74.295 98.425) (width 0.25) (layer "F.Cu") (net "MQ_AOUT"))
 (segment (start 75.565 97) (end 75.565 97.155) (width 0.25) (layer "F.Cu") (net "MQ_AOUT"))
 (segment (start 75.93 108.26) (end 75.93 100.06) (width 0.25) (layer "F.Cu") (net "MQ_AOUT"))
 (segment (start 74.5 109) (end 75.19 109) (width 0.25) (layer "F.Cu") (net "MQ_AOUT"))
 (segment (start 78.256701 97.06) (end 75.625 97.06) (width 0.25) (layer "F.Cu") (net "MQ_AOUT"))
 (segment (start 79.621701 98.425) (end 78.256701 97.06) (width 0.25) (layer "F.Cu") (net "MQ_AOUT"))
 (segment (start 80.5 98.425) (end 79.621701 98.425) (width 0.25) (layer "F.Cu") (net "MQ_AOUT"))
 (segment (start 87.88 82.5) (end 85.925 84.455) (width 0.25) (layer "F.Cu") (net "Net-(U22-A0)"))
 (segment (start 72.39 104.89) (end 73.545 106.045) (width 0.25) (layer "F.Cu") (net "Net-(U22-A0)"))
 (segment (start 73.545 106.045) (end 74.295 106.045) (width 0.25) (layer "F.Cu") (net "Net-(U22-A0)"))
 (segment (start 85.925 84.455) (end 75.565 84.455) (width 0.25) (layer "F.Cu") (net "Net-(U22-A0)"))
 (segment (start 72.39 87.63) (end 72.39 104.89) (width 0.25) (layer "F.Cu") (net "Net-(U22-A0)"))
 (segment (start 75.565 84.455) (end 72.39 87.63) (width 0.25) (layer "F.Cu") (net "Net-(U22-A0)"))
 (segment (start 107.87 74.93) (end 111.045 78.105) (width 0.25) (layer "F.Cu") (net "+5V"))
 (segment (start 95.5 74.93) (end 107.87 74.93) (width 0.25) (layer "F.Cu") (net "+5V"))
 (segment (start 86.375 101.858299) (end 86.375 103.46) (width 0.25) (layer "F.Cu") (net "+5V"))
 (segment (start 87 102.5) (end 95 102.5) (width 0.25) (layer "F.Cu") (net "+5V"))
 (segment (start 113.1062 90.805) (end 111.045 88.7438) (width 0.25) (layer "F.Cu") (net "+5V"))
 (segment (start 111.045 78.105) (end 111.045 88.7438) (width 0.25) (layer "F.Cu") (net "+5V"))
 (segment (start 95.5 82.5) (end 95.5 74.93) (width 0.25) (layer "F.Cu") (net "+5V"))
 (segment (start 113.1062 90.805) (end 121.92 90.805) (width 0.25) (layer "F.Cu") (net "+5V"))
 (via (at 95 102.5) (size 0.6) (drill 0.3) (layers "F.Cu" "B.Cu") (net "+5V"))
 (segment (start 95.5 102) (end 95.5 82.5) (width 0.25) (layer "B.Cu") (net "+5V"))
 (segment (start 95 102.5) (end 95.5 102) (width 0.25) (layer "B.Cu") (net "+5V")))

